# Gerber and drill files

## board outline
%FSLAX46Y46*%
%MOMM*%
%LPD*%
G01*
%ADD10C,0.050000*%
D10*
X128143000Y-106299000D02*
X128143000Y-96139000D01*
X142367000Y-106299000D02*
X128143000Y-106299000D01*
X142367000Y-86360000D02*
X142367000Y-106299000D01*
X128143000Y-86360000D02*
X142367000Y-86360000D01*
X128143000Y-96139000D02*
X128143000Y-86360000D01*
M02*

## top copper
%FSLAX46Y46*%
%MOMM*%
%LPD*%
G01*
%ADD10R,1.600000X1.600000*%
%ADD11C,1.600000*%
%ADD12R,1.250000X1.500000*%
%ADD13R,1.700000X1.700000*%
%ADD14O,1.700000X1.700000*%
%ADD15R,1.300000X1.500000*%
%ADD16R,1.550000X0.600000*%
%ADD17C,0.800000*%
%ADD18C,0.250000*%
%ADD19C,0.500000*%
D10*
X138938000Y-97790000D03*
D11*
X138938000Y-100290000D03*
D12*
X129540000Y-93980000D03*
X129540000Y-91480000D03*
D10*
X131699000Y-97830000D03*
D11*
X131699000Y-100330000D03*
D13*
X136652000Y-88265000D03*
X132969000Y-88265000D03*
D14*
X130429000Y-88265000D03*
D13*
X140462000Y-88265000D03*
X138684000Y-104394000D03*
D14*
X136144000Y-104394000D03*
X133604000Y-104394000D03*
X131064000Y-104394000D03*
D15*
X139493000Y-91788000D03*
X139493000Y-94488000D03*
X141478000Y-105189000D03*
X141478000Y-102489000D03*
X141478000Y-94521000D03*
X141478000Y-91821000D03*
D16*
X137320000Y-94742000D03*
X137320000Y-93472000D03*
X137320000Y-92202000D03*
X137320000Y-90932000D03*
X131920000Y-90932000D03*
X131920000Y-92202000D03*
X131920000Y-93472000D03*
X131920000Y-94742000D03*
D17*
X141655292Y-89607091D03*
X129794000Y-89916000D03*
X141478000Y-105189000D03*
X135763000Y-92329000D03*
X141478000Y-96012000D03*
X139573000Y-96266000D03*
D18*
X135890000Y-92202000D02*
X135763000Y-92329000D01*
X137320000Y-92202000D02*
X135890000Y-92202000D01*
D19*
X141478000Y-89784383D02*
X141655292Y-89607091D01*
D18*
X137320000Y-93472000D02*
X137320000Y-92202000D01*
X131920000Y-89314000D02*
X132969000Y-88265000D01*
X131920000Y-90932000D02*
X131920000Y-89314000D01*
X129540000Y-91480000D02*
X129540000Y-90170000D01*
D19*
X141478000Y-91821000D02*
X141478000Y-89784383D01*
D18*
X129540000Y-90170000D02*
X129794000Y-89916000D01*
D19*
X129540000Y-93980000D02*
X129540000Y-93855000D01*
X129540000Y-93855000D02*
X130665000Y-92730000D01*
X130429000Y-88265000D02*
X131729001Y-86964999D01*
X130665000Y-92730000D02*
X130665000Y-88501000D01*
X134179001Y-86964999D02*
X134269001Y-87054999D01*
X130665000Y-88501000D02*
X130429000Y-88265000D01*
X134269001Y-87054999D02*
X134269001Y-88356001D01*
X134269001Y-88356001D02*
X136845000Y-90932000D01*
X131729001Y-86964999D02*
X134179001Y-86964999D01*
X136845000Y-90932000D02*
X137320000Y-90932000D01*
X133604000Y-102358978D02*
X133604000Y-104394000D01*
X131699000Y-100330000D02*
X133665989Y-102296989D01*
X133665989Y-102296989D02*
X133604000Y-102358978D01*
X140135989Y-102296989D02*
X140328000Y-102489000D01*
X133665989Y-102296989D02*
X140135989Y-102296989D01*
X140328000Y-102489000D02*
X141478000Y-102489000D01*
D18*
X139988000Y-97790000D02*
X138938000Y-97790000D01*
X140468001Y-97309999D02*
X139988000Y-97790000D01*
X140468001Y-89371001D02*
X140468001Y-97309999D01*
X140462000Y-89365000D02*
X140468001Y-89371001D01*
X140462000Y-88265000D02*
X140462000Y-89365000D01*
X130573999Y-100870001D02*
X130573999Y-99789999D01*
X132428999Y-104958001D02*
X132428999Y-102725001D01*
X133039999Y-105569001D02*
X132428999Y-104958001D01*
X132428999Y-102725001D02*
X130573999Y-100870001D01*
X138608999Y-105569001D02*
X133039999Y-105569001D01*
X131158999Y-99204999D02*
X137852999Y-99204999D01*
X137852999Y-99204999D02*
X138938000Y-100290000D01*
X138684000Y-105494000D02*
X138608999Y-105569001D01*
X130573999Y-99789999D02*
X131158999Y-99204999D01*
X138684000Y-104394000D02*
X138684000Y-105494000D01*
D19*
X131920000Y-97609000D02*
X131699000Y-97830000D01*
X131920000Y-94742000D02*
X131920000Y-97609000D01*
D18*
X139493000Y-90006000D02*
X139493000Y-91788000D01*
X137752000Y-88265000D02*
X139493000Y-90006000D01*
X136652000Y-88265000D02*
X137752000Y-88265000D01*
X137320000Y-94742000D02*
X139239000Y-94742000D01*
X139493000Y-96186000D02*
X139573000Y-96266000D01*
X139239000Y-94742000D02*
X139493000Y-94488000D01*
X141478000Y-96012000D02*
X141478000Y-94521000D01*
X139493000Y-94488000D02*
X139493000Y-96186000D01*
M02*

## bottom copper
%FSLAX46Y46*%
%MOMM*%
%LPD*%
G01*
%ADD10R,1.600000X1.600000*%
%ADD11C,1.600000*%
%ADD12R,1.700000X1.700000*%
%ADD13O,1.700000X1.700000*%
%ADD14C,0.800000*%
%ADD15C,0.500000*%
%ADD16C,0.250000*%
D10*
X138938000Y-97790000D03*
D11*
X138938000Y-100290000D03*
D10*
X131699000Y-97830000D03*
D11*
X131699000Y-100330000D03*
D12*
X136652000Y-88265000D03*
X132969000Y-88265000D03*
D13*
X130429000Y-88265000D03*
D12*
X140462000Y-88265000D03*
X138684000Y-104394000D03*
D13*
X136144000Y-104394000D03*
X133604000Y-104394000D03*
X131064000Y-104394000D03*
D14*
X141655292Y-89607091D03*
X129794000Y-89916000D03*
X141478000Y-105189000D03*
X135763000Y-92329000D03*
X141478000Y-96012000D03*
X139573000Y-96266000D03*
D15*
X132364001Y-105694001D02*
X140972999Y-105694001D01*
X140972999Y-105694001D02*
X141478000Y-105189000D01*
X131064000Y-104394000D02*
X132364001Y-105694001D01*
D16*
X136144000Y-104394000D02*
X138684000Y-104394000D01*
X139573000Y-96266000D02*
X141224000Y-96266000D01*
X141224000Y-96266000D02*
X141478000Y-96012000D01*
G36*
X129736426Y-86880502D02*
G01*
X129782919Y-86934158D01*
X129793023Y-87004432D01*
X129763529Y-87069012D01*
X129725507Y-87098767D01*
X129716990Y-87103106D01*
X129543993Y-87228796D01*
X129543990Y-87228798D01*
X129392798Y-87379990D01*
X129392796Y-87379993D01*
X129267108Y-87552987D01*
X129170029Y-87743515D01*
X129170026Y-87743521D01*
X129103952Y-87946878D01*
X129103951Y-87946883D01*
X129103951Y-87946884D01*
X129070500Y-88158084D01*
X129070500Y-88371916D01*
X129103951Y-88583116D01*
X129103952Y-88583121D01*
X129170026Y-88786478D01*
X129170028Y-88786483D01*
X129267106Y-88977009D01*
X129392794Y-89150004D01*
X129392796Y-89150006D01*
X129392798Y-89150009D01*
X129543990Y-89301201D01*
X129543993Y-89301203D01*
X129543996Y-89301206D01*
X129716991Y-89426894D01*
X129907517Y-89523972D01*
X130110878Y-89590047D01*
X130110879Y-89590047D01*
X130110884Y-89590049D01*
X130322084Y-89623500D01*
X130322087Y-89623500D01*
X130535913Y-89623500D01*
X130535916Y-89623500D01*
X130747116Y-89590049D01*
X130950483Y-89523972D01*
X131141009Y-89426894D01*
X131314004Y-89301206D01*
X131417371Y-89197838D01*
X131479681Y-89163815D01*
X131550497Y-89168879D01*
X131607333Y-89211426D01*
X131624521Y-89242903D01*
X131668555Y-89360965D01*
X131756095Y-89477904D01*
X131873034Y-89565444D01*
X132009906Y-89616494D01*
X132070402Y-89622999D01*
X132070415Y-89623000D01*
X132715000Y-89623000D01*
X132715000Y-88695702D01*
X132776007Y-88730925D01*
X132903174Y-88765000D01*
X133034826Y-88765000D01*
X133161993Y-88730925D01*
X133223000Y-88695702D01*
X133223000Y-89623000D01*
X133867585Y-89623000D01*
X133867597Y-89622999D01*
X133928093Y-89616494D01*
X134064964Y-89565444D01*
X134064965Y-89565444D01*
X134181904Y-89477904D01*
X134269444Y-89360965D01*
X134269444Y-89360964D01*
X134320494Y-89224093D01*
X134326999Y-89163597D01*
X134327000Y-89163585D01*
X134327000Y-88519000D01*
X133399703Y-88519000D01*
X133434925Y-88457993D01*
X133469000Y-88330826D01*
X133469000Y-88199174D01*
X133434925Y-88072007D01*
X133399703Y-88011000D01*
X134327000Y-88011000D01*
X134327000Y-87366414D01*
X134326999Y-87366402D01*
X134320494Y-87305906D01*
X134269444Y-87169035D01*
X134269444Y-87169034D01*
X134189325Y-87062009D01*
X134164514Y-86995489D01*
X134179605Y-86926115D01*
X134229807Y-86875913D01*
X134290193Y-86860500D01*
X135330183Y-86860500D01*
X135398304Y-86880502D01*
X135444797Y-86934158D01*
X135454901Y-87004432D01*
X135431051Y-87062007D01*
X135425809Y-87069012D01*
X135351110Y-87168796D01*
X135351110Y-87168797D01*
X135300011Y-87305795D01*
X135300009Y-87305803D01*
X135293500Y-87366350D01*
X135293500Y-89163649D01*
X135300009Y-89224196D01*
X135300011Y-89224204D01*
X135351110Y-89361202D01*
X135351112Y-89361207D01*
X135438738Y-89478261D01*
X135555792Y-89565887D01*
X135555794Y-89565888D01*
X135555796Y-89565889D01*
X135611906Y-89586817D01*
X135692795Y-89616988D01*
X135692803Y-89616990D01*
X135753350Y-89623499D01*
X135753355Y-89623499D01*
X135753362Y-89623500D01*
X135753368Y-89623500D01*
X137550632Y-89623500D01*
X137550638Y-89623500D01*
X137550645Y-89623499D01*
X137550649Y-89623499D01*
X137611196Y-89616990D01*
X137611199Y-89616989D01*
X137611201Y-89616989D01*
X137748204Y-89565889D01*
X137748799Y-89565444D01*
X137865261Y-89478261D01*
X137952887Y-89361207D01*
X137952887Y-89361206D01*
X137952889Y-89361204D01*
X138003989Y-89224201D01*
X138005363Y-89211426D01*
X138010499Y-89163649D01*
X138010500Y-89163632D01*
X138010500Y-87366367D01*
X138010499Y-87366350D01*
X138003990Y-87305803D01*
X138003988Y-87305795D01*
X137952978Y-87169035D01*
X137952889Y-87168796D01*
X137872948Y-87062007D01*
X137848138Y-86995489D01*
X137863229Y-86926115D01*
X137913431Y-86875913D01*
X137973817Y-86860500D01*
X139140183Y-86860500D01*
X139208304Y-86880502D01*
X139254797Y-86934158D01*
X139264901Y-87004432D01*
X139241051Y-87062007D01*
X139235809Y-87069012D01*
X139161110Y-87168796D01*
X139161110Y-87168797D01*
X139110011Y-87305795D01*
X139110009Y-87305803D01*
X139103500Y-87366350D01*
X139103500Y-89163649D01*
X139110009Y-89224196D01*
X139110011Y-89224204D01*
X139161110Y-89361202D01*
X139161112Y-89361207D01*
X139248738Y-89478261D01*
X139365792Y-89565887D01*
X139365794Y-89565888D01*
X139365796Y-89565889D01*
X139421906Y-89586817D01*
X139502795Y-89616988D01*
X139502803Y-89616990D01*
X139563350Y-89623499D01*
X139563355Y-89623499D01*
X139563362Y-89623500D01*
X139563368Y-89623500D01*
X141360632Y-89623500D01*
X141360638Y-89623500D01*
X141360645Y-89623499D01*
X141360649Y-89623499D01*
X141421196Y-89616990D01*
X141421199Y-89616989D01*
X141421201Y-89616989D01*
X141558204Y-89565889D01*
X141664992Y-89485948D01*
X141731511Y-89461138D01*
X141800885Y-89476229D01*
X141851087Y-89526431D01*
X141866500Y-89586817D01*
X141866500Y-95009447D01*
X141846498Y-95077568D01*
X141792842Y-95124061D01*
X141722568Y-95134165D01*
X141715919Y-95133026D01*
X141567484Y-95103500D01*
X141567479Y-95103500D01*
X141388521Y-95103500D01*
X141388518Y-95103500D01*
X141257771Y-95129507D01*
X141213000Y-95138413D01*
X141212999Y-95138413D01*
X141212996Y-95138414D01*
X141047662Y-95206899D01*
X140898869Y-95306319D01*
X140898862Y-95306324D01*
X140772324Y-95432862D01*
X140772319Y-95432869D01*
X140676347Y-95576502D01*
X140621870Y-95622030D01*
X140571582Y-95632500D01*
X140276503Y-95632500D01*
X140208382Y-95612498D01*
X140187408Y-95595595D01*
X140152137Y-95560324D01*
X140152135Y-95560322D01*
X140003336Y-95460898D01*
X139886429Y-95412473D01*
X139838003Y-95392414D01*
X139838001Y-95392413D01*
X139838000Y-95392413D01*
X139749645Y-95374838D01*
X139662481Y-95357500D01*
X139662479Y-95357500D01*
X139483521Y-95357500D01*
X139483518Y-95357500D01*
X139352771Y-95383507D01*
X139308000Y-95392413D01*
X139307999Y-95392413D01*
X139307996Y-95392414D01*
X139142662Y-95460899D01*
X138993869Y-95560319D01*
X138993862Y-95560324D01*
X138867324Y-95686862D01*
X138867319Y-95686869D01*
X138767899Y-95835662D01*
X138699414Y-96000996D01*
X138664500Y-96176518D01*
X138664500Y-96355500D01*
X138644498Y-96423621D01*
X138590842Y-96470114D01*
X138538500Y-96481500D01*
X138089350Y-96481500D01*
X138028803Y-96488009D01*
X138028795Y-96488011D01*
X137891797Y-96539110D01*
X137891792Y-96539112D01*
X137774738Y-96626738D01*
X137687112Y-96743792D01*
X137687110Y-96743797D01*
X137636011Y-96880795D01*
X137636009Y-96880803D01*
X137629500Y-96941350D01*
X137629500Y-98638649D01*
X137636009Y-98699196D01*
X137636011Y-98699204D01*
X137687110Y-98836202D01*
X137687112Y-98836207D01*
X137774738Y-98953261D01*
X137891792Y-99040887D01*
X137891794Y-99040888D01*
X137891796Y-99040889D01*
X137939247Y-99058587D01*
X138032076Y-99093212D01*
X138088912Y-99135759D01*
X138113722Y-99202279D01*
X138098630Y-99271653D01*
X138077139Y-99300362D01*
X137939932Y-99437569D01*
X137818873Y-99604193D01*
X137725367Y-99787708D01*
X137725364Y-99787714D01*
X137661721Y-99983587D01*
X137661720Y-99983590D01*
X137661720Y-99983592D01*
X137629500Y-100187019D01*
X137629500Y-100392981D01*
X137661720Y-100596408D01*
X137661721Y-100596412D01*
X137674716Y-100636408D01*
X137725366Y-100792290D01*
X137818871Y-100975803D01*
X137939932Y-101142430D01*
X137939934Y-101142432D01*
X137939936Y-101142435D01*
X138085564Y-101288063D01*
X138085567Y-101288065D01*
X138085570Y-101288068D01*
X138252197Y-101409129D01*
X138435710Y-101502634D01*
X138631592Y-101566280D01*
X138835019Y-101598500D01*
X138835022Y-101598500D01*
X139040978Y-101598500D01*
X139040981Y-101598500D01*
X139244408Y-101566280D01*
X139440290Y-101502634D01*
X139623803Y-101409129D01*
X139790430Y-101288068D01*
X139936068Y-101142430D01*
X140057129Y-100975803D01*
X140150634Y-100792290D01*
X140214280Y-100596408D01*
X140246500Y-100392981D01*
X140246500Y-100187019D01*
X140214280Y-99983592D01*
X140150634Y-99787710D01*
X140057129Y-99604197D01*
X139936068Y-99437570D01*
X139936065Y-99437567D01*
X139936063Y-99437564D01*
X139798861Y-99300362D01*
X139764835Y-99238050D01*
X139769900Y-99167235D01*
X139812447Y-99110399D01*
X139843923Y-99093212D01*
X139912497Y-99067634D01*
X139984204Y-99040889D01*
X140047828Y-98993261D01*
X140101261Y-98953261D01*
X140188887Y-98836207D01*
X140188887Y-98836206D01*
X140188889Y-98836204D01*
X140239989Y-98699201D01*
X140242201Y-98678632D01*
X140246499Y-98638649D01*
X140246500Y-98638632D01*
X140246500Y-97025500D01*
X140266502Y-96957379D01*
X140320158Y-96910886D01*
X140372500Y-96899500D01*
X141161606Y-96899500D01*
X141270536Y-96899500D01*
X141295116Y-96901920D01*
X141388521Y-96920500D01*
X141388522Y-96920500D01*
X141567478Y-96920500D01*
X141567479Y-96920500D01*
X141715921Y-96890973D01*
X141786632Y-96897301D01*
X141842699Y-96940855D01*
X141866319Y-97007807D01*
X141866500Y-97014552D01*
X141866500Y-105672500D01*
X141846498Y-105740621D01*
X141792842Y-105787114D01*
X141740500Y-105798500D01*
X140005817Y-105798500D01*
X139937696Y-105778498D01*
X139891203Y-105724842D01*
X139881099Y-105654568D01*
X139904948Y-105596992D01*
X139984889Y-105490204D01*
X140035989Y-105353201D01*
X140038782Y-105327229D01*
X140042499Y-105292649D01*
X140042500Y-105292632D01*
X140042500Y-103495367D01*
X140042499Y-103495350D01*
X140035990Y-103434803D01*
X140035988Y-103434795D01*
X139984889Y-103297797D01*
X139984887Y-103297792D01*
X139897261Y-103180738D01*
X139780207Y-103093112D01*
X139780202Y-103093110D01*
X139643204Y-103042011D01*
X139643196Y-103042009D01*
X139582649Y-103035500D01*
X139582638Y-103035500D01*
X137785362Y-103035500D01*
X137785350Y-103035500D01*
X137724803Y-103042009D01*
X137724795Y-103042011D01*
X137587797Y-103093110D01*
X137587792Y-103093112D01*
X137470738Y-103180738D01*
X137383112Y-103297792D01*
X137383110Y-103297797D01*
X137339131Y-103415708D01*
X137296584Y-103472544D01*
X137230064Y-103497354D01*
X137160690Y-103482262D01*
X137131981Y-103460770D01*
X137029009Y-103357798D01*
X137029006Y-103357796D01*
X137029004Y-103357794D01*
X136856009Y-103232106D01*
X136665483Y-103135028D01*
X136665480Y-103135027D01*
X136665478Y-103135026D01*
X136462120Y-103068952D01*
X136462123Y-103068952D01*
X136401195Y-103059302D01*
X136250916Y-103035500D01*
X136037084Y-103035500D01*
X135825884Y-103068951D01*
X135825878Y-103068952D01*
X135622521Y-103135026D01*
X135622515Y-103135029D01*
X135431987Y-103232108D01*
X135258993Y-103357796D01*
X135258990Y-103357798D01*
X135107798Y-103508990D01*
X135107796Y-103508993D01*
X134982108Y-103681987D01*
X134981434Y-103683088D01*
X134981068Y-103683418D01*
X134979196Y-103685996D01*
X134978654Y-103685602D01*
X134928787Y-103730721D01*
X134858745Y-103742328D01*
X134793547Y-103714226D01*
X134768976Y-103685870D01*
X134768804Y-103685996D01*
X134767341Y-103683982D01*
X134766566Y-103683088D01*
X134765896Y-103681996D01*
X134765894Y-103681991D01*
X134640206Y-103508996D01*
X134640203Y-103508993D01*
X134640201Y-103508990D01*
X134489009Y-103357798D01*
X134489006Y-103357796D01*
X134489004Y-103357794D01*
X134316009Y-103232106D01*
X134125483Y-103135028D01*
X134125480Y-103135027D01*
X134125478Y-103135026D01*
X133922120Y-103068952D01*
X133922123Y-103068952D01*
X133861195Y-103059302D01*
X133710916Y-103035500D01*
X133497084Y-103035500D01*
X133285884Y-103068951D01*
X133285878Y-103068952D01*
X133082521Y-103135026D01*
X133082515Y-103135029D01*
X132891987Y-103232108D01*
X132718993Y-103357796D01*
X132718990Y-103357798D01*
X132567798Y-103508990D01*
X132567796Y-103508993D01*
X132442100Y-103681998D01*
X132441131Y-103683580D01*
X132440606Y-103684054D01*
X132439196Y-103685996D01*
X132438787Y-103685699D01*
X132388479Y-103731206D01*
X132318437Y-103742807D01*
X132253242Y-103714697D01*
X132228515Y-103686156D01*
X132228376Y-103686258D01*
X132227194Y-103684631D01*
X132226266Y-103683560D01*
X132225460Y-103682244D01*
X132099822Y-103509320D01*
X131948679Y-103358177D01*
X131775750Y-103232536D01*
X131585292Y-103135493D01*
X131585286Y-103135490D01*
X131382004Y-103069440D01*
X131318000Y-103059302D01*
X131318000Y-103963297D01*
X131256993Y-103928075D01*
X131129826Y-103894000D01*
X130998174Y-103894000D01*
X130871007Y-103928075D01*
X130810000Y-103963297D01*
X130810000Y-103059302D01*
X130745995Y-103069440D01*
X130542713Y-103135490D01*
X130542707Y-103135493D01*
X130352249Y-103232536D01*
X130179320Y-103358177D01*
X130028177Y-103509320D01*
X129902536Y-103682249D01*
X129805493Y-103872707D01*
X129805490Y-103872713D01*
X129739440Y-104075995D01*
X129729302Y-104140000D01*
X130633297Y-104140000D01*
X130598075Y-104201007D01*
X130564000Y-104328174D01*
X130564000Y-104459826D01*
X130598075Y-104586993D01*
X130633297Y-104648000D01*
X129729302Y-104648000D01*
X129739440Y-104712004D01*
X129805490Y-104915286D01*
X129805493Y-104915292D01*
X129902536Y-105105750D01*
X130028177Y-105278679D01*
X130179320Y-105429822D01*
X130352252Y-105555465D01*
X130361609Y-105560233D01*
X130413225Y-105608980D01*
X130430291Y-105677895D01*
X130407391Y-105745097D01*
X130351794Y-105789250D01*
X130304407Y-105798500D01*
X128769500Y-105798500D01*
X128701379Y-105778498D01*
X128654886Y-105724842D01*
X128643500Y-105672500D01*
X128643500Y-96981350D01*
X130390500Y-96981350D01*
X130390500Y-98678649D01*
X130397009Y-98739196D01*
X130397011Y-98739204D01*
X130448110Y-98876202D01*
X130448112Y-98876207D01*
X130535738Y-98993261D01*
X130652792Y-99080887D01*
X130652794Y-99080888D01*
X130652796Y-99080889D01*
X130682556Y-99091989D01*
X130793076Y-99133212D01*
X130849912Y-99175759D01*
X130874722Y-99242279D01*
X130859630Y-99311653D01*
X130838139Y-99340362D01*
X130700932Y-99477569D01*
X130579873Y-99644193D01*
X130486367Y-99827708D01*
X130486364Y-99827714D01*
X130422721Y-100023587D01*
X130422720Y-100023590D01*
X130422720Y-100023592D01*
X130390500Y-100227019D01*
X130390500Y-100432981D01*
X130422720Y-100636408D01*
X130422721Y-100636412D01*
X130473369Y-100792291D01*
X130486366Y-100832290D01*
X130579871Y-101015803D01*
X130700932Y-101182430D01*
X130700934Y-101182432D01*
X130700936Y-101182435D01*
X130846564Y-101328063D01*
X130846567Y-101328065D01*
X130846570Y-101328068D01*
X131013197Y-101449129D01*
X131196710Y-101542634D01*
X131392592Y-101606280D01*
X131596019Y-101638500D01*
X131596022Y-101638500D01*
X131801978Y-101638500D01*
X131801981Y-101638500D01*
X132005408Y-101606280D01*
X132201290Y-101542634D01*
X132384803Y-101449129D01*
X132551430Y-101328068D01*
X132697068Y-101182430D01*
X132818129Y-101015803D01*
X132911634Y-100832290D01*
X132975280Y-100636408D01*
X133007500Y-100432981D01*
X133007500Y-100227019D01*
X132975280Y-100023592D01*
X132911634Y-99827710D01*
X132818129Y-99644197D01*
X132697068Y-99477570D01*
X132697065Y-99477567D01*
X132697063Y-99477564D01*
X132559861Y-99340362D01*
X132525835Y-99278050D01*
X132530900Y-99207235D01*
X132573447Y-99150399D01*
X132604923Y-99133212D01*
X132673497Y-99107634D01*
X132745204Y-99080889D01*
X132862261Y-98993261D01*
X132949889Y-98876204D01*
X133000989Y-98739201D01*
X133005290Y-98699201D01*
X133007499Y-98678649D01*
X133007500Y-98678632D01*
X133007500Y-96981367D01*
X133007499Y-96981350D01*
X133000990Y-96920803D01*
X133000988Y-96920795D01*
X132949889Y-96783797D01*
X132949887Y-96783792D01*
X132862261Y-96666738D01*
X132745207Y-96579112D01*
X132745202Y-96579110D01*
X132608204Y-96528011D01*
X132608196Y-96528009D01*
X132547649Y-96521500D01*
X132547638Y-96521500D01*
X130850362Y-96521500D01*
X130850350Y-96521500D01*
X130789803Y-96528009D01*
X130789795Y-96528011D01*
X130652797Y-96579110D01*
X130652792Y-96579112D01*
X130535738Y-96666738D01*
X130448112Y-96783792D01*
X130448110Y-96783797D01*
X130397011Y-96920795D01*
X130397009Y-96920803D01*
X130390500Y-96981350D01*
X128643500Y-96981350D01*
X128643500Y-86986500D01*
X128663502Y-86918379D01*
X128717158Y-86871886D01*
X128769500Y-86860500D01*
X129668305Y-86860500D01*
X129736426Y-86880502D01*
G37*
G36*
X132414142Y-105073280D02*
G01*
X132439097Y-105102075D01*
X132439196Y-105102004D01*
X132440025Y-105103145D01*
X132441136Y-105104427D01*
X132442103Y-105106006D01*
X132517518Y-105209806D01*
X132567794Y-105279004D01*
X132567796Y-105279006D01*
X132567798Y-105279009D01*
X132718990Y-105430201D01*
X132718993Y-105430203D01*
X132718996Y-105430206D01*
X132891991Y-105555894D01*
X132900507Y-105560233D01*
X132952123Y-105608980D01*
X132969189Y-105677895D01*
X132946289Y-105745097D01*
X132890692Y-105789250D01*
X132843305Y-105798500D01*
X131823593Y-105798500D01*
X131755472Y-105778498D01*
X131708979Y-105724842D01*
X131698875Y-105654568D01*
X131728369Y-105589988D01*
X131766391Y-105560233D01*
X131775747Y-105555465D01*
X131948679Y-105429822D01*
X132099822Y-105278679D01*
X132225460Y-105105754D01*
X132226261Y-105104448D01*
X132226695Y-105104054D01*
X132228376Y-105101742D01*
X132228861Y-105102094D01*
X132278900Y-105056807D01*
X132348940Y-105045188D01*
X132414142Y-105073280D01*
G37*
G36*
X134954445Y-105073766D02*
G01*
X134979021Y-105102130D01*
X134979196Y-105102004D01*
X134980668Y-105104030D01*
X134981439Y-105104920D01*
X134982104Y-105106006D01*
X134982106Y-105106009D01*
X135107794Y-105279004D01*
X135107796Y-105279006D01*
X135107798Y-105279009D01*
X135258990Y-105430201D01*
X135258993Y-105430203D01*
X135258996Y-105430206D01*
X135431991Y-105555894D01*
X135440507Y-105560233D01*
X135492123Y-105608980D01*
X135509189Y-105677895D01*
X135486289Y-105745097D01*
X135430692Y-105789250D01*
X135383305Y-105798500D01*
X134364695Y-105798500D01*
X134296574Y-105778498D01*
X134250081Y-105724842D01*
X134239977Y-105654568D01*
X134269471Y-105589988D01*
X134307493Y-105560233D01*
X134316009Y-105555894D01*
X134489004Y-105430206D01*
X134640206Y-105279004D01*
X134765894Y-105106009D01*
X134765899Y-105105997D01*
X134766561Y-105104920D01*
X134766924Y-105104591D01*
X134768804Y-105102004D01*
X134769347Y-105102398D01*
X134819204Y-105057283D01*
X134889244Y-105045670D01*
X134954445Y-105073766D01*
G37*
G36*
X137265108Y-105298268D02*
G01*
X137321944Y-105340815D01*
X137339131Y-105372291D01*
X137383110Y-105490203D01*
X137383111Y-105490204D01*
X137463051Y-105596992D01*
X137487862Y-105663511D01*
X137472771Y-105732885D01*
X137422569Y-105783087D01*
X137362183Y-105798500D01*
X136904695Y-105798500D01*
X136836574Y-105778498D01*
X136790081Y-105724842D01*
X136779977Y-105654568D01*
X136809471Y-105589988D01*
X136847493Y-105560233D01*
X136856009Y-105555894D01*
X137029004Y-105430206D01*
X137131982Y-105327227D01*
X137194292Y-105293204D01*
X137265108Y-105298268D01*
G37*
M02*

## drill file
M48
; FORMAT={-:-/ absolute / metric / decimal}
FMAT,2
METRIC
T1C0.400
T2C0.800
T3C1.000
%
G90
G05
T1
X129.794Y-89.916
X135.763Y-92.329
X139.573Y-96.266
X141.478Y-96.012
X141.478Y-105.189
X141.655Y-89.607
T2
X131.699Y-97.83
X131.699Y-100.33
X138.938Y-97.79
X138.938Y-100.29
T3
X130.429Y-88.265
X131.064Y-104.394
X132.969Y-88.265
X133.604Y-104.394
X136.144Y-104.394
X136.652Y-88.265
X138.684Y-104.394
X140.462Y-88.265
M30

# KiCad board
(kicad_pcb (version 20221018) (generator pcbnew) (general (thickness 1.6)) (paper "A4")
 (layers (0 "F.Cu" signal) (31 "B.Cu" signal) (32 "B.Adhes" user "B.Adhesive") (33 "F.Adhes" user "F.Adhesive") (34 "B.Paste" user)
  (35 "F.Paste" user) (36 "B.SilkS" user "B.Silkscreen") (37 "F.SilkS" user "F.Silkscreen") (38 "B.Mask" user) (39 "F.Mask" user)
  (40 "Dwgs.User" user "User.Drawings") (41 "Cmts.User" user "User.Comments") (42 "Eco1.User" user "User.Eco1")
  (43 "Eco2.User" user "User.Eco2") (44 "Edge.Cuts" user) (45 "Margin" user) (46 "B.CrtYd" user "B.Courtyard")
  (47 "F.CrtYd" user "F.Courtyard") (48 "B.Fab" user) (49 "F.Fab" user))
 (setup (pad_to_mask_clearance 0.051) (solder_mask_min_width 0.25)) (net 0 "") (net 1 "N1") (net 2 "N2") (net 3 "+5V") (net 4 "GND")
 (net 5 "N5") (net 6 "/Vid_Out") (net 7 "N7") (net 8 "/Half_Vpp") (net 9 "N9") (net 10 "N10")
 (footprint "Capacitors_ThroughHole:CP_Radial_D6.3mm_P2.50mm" (layer "F.Cu") (at 138.938 97.79 -90)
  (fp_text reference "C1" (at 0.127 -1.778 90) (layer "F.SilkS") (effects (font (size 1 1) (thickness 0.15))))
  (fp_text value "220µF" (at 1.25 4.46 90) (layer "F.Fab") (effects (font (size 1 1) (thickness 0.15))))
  (pad "1" thru_hole rect (at 0 0 270) (size 1.6 1.6) (drill 0.8) (layers "*.Cu" "*.Mask") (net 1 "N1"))
  (pad "2" thru_hole circle (at 2.5 0 270) (size 1.6 1.6) (drill 0.8) (layers "*.Cu" "*.Mask") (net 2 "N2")))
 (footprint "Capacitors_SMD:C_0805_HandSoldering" (layer "F.Cu") (at 129.54 92.73 90)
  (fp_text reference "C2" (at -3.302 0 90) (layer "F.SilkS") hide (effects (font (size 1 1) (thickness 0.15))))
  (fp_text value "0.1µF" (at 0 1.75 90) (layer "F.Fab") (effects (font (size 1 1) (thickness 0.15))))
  (pad "1" smd rect (at -1.25 0 90) (size 1.5 1.25) (layers "F.Cu" "F.Paste" "F.Mask") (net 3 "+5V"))
  (pad "2" smd rect (at 1.25 0 90) (size 1.5 1.25) (layers "F.Cu" "F.Paste" "F.Mask") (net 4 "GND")))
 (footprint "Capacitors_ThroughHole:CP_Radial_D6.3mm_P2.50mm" (layer "F.Cu") (at 131.699 97.83 -90)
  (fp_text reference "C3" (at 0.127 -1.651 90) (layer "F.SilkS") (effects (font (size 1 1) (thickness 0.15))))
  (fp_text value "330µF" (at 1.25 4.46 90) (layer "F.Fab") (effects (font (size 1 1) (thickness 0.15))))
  (pad "1" thru_hole rect (at 0 0 270) (size 1.6 1.6) (drill 0.8) (layers "*.Cu" "*.Mask") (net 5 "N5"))
  (pad "2" thru_hole circle (at 2.5 0 270) (size 1.6 1.6) (drill 0.8) (layers "*.Cu" "*.Mask") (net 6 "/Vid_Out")))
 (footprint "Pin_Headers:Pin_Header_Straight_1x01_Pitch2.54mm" (layer "F.Cu") (at 136.652 88.265)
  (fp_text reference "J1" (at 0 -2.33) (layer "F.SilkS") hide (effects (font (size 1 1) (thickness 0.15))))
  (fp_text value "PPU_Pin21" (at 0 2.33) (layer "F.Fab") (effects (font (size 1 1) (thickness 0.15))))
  (pad "1" thru_hole rect (at 0 0) (size 1.7 1.7) (drill 1) (layers "*.Cu" "*.Mask") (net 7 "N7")))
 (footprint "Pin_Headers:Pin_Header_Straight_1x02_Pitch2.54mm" (layer "F.Cu") (at 132.969 88.265 -90)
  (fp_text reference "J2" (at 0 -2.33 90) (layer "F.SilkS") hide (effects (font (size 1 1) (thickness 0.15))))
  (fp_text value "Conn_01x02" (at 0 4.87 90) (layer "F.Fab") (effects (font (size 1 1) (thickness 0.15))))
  (pad "1" thru_hole rect (at 0 0 270) (size 1.7 1.7) (drill 1) (layers "*.Cu" "*.Mask") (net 4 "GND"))
  (pad "2" thru_hole oval (at 0 2.54 270) (size 1.7 1.7) (drill 1) (layers "*.Cu" "*.Mask") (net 3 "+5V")))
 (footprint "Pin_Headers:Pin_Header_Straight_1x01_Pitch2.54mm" (layer "F.Cu") (at 140.462 88.265)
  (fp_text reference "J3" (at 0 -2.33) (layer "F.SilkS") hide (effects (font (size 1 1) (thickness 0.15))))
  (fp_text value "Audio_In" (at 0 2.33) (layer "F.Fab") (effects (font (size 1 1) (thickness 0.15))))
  (pad "1" thru_hole rect (at 0 0) (size 1.7 1.7) (drill 1) (layers "*.Cu" "*.Mask") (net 1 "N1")))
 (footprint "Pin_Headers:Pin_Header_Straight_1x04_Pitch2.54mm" (layer "F.Cu") (at 138.684 104.394 -90)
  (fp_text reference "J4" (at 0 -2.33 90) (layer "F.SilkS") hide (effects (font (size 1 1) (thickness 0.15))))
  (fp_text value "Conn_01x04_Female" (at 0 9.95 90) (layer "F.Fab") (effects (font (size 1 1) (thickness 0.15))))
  (pad "1" thru_hole rect (at 0 0 270) (size 1.7 1.7) (drill 1) (layers "*.Cu" "*.Mask") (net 2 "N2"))
  (pad "2" thru_hole oval (at 0 2.54 270) (size 1.7 1.7) (drill 1) (layers "*.Cu" "*.Mask") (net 2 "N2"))
  (pad "3" thru_hole oval (at 0 5.08 270) (size 1.7 1.7) (drill 1) (layers "*.Cu" "*.Mask") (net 6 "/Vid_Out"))
  (pad "4" thru_hole oval (at 0 7.62 270) (size 1.7 1.7) (drill 1) (layers "*.Cu" "*.Mask") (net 4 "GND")))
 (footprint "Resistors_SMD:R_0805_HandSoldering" (layer "F.Cu") (at 139.493 93.138 -90)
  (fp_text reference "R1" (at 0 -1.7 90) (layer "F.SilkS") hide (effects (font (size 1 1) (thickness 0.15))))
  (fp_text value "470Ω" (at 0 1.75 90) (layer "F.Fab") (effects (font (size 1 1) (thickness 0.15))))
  (pad "1" smd rect (at -1.35 0 270) (size 1.5 1.3) (layers "F.Cu" "F.Paste" "F.Mask") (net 7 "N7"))
  (pad "2" smd rect (at 1.35 0 270) (size 1.5 1.3) (layers "F.Cu" "F.Paste" "F.Mask") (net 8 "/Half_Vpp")))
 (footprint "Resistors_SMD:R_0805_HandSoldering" (layer "F.Cu") (at 141.478 103.839 90)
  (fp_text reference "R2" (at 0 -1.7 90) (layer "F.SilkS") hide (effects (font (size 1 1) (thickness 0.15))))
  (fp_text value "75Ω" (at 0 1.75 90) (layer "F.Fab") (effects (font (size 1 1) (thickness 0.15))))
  (pad "1" smd rect (at -1.35 0 90) (size 1.5 1.3) (layers "F.Cu" "F.Paste" "F.Mask") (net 4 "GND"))
  (pad "2" smd rect (at 1.35 0 90) (size 1.5 1.3) (layers "F.Cu" "F.Paste" "F.Mask") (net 6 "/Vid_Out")))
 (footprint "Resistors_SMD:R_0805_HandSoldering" (layer "F.Cu") (at 141.478 93.171 90)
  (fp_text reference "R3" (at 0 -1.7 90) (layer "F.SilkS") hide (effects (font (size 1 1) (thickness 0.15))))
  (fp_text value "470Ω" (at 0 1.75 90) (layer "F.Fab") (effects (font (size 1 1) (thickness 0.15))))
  (pad "1" smd rect (at -1.35 0 90) (size 1.5 1.3) (layers "F.Cu" "F.Paste" "F.Mask") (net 8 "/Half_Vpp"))
  (pad "2" smd rect (at 1.35 0 90) (size 1.5 1.3) (layers "F.Cu" "F.Paste" "F.Mask") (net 4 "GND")))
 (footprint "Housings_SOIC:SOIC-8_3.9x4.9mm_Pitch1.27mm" (layer "F.Cu") (at 134.62 92.837 180)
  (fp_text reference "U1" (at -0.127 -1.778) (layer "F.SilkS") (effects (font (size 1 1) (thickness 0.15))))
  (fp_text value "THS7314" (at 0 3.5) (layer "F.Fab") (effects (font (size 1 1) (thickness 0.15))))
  (pad "1" smd rect (at -2.7 -1.905 180) (size 1.55 0.6) (layers "F.Cu" "F.Paste" "F.Mask") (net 8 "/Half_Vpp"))
  (pad "2" smd rect (at -2.7 -0.635 180) (size 1.55 0.6) (layers "F.Cu" "F.Paste" "F.Mask") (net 4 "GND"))
  (pad "3" smd rect (at -2.7 0.635 180) (size 1.55 0.6) (layers "F.Cu" "F.Paste" "F.Mask") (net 4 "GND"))
  (pad "4" smd rect (at -2.7 1.905 180) (size 1.55 0.6) (layers "F.Cu" "F.Paste" "F.Mask") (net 3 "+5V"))
  (pad "5" smd rect (at 2.7 1.905 180) (size 1.55 0.6) (layers "F.Cu" "F.Paste" "F.Mask") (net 4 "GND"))
  (pad "6" smd rect (at 2.7 0.635 180) (size 1.55 0.6) (layers "F.Cu" "F.Paste" "F.Mask") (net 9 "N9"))
  (pad "7" smd rect (at 2.7 -0.635 180) (size 1.55 0.6) (layers "F.Cu" "F.Paste" "F.Mask") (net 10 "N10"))
  (pad "8" smd rect (at 2.7 -1.905 180) (size 1.55 0.6) (layers "F.Cu" "F.Paste" "F.Mask") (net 5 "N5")))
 (gr_line (start 128.143 106.299) (end 128.143 96.139) (stroke (width 0.05) (type solid)) (layer "Edge.Cuts"))
 (gr_line (start 142.367 106.299) (end 128.143 106.299) (stroke (width 0.05) (type solid)) (layer "Edge.Cuts"))
 (gr_line (start 142.367 86.36) (end 142.367 106.299) (stroke (width 0.05) (type solid)) (layer "Edge.Cuts"))
 (gr_line (start 128.143 86.36) (end 142.367 86.36) (stroke (width 0.05) (type solid)) (layer "Edge.Cuts"))
 (gr_line (start 128.143 96.139) (end 128.143 86.36) (stroke (width 0.05) (type solid)) (layer "Edge.Cuts"))
 (segment (start 135.89 92.202) (end 135.763 92.329) (width 0.25) (layer "F.Cu") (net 4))
 (segment (start 137.32 92.202) (end 135.89 92.202) (width 0.25) (layer "F.Cu") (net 4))
 (segment (start 141.478 89.784383) (end 141.655292 89.607091) (width 0.5) (layer "F.Cu") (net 4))
 (segment (start 137.32 93.472) (end 137.32 92.202) (width 0.25) (layer "F.Cu") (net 4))
 (segment (start 131.92 89.314) (end 132.969 88.265) (width 0.25) (layer "F.Cu") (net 4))
 (segment (start 131.92 90.932) (end 131.92 89.314) (width 0.25) (layer "F.Cu") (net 4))
 (segment (start 129.54 91.48) (end 129.54 90.17) (width 0.25) (layer "F.Cu") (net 4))
 (segment (start 141.478 91.821) (end 141.478 89.784383) (width 0.5) (layer "F.Cu") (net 4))
 (segment (start 129.54 90.17) (end 129.794 89.916) (width 0.25) (layer "F.Cu") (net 4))
 (via (at 141.655292 89.607091) (size 0.8) (drill 0.4) (layers "F.Cu" "B.Cu") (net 4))
 (via (at 129.794 89.916) (size 0.8) (drill 0.4) (layers "F.Cu" "B.Cu") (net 4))
 (via (at 141.478 105.189) (size 0.8) (drill 0.4) (layers "F.Cu" "B.Cu") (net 4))
 (via (at 135.763 92.329) (size 0.8) (drill 0.4) (layers "F.Cu" "B.Cu") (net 4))
 (segment (start 132.364001 105.694001) (end 140.972999 105.694001) (width 0.5) (layer "B.Cu") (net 4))
 (segment (start 140.972999 105.694001) (end 141.478 105.189) (width 0.5) (layer "B.Cu") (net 4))
 (segment (start 131.064 104.394) (end 132.364001 105.694001) (width 0.5) (layer "B.Cu") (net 4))
 (segment (start 129.54 93.98) (end 129.54 93.855) (width 0.5) (layer "F.Cu") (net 3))
 (segment (start 129.54 93.855) (end 130.665 92.73) (width 0.5) (layer "F.Cu") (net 3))
 (segment (start 130.429 88.265) (end 131.729001 86.964999) (width 0.5) (layer "F.Cu") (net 3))
 (segment (start 130.665 92.73) (end 130.665 88.501) (width 0.5) (layer "F.Cu") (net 3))
 (segment (start 134.179001 86.964999) (end 134.269001 87.054999) (width 0.5) (layer "F.Cu") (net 3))
 (segment (start 130.665 88.501) (end 130.429 88.265) (width 0.5) (layer "F.Cu") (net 3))
 (segment (start 134.269001 87.054999) (end 134.269001 88.356001) (width 0.5) (layer "F.Cu") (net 3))
 (segment (start 134.269001 88.356001) (end 136.845 90.932) (width 0.5) (layer "F.Cu") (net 3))
 (segment (start 131.729001 86.964999) (end 134.179001 86.964999) (width 0.5) (layer "F.Cu") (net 3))
 (segment (start 136.845 90.932) (end 137.32 90.932) (width 0.5) (layer "F.Cu") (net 3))
 (segment (start 133.604 102.358978) (end 133.604 104.394) (width 0.5) (layer "F.Cu") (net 6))
 (segment (start 131.699 100.33) (end 133.665989 102.296989) (width 0.5) (layer "F.Cu") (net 6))
 (segment (start 133.665989 102.296989) (end 133.604 102.358978) (width 0.5) (layer "F.Cu") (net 6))
 (segment (start 140.135989 102.296989) (end 140.328 102.489) (width 0.5) (layer "F.Cu") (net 6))
 (segment (start 133.665989 102.296989) (end 140.135989 102.296989) (width 0.5) (layer "F.Cu") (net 6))
 (segment (start 140.328 102.489) (end 141.478 102.489) (width 0.5) (layer "F.Cu") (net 6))
 (segment (start 139.988 97.79) (end 138.938 97.79) (width 0.25) (layer "F.Cu") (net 1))
 (segment (start 140.468001 97.309999) (end 139.988 97.79) (width 0.25) (layer "F.Cu") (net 1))
 (segment (start 140.468001 89.371001) (end 140.468001 97.309999) (width 0.25) (layer "F.Cu") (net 1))
 (segment (start 140.462 89.365) (end 140.468001 89.371001) (width 0.25) (layer "F.Cu") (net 1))
 (segment (start 140.462 88.265) (end 140.462 89.365) (width 0.25) (layer "F.Cu") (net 1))
 (segment (start 130.573999 100.870001) (end 130.573999 99.789999) (width 0.25) (layer "F.Cu") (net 2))
 (segment (start 132.428999 104.958001) (end 132.428999 102.725001) (width 0.25) (layer "F.Cu") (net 2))
 (segment (start 133.039999 105.569001) (end 132.428999 104.958001) (width 0.25) (layer "F.Cu") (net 2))
 (segment (start 132.428999 102.725001) (end 130.573999 100.870001) (width 0.25) (layer "F.Cu") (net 2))
 (segment (start 138.608999 105.569001) (end 133.039999 105.569001) (width 0.25) (layer "F.Cu") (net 2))
 (segment (start 131.158999 99.204999) (end 137.852999 99.204999) (width 0.25) (layer "F.Cu") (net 2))
 (segment (start 137.852999 99.204999) (end 138.938 100.29) (width 0.25) (layer "F.Cu") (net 2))
 (segment (start 138.684 105.494) (end 138.608999 105.569001) (width 0.25) (layer "F.Cu") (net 2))
 (segment (start 130.573999 99.789999) (end 131.158999 99.204999) (width 0.25) (layer "F.Cu") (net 2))
 (segment (start 138.684 104.394) (end 138.684 105.494) (width 0.25) (layer "F.Cu") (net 2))
 (segment (start 136.144 104.394) (end 138.684 104.394) (width 0.25) (layer "B.Cu") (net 2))
 (segment (start 131.92 97.609) (end 131.699 97.83) (width 0.5) (layer "F.Cu") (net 5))
 (segment (start 131.92 94.742) (end 131.92 97.609) (width 0.5) (layer "F.Cu") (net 5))
 (segment (start 139.493 90.006) (end 139.493 91.788) (width 0.25) (layer "F.Cu") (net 7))
 (segment (start 137.752 88.265) (end 139.493 90.006) (width 0.25) (layer "F.Cu") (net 7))
 (segment (start 136.652 88.265) (end 137.752 88.265) (width 0.25) (layer "F.Cu") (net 7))
 (segment (start 137.32 94.742) (end 139.239 94.742) (width 0.25) (layer "F.Cu") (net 8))
 (segment (start 139.493 96.186) (end 139.573 96.266) (width 0.25) (layer "F.Cu") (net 8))
 (segment (start 139.239 94.742) (end 139.493 94.488) (width 0.25) (layer "F.Cu") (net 8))
 (segment (start 141.478 96.012) (end 141.478 94.521) (width 0.25) (layer "F.Cu") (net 8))
 (segment (start 139.493 94.488) (end 139.493 96.186) (width 0.25) (layer "F.Cu") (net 8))
 (via (at 141.478 96.012) (size 0.8) (drill 0.4) (layers "F.Cu" "B.Cu") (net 8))
 (via (at 139.573 96.266) (size 0.8) (drill 0.4) (layers "F.Cu" "B.Cu") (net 8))
 (segment (start 139.573 96.266) (end 141.224 96.266) (width 0.25) (layer "B.Cu") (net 8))
 (segment (start 141.224 96.266) (end 141.478 96.012) (width 0.25) (layer "B.Cu") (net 8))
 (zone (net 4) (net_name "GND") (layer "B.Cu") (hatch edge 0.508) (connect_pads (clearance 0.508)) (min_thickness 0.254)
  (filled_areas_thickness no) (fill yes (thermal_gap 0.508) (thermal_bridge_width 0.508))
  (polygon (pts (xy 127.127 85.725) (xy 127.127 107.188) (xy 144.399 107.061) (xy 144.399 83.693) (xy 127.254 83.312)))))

